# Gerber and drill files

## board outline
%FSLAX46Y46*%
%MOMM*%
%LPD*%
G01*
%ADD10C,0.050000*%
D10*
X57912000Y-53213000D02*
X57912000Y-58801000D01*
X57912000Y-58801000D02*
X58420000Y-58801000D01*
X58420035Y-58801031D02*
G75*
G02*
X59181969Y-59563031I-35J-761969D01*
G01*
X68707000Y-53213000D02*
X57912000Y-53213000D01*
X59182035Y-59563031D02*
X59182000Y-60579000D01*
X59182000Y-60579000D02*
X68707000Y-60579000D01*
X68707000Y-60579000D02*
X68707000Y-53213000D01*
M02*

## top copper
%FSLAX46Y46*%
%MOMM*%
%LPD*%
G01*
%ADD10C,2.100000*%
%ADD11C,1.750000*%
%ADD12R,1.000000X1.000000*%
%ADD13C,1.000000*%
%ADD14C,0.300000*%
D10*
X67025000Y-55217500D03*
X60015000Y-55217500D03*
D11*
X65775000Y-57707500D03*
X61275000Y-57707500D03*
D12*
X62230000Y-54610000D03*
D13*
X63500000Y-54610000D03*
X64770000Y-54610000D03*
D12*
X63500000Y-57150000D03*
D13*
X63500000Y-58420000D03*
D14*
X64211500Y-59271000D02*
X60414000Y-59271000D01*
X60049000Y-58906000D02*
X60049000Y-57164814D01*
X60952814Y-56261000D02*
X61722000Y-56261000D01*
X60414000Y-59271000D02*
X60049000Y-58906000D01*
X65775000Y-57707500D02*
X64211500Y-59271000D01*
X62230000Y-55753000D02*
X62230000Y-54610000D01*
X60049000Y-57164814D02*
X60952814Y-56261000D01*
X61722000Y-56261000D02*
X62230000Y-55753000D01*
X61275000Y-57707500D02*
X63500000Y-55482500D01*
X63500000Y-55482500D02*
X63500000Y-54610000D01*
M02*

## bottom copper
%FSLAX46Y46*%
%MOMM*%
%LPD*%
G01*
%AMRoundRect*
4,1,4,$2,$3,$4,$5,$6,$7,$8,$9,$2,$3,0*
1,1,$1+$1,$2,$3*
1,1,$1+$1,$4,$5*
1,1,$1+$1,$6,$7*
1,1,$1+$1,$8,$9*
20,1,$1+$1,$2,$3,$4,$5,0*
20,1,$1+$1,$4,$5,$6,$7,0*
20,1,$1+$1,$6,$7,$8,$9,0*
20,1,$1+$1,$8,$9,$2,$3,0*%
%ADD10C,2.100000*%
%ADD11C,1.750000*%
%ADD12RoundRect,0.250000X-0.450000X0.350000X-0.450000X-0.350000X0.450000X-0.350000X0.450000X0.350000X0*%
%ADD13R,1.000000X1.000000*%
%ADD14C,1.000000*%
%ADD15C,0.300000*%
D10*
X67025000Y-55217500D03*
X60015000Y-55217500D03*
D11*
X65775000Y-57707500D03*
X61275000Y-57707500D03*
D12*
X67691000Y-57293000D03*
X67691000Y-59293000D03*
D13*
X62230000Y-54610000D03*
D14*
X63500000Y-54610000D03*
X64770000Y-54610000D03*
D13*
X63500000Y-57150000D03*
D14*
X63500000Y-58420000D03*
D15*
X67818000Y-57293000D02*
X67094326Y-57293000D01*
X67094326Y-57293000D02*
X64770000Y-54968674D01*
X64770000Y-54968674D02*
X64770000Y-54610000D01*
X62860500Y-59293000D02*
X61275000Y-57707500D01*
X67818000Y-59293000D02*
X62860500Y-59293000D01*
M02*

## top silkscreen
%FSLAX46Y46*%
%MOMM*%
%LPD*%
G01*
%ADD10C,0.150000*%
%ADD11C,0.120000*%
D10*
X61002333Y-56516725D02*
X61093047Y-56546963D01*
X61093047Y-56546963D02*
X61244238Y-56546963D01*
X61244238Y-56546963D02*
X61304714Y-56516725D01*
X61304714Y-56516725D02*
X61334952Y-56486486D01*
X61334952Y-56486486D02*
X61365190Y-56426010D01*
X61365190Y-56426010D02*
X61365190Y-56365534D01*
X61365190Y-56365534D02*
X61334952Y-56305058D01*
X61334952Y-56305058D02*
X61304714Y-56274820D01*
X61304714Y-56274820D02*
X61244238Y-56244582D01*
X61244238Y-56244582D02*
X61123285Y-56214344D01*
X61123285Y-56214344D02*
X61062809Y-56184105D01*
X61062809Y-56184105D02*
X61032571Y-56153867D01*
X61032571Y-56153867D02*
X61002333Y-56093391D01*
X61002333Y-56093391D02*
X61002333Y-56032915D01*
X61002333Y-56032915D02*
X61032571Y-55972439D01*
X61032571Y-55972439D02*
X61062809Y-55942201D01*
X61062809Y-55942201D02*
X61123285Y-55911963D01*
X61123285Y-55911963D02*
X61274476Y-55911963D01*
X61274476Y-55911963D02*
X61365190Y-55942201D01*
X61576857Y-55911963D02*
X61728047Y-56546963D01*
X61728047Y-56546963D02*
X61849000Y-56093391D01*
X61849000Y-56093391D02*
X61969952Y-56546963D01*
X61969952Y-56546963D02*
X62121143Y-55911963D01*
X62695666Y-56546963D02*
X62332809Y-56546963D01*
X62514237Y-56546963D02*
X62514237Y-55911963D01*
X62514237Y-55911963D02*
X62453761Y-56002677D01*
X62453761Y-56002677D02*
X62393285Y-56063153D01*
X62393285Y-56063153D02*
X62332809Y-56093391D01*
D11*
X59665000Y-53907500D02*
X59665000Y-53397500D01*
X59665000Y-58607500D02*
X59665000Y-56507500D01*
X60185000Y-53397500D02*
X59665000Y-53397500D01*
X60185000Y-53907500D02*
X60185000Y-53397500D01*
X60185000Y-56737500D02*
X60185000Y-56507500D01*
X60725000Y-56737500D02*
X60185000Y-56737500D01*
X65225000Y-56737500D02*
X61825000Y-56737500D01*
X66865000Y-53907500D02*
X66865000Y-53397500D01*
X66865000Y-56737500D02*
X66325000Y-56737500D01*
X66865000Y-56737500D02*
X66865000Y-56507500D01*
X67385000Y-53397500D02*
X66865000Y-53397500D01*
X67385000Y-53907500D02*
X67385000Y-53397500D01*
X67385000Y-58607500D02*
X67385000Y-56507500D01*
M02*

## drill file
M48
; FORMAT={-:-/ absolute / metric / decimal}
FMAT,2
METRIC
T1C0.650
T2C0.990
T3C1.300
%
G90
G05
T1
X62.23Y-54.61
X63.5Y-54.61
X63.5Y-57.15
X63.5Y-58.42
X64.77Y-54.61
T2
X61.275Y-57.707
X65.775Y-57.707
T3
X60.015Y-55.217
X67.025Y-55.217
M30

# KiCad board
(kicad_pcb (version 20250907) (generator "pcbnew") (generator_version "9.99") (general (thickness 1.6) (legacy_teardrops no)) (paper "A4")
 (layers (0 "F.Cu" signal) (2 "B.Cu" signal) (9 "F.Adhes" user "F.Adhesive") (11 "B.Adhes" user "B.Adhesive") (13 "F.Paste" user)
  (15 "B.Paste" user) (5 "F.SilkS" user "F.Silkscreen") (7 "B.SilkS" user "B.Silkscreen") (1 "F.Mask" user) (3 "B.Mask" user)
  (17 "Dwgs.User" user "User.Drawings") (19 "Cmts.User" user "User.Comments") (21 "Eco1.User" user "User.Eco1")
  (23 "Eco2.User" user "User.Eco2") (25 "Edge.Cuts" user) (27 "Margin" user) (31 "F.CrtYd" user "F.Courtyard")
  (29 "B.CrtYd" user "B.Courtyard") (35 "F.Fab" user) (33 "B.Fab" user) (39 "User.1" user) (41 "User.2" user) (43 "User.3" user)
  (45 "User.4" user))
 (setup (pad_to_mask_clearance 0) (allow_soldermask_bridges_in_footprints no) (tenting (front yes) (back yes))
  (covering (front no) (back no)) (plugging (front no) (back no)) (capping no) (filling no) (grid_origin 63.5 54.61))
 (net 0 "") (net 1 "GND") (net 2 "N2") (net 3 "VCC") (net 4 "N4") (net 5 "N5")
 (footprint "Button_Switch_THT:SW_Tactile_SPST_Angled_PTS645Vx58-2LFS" (layer "F.Cu") (at 65.775 57.7075 180)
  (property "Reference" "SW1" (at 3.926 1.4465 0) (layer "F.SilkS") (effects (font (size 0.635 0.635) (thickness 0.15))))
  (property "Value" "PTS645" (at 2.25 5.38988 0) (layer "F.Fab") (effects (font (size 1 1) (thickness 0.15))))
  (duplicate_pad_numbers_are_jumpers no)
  (fp_line (start 6.11 3.8) (end 6.11 4.31) (stroke (width 0.12) (type solid)) (layer "F.SilkS"))
  (fp_line (start 6.11 -0.9) (end 6.11 1.2) (stroke (width 0.12) (type solid)) (layer "F.SilkS"))
  (fp_line (start 5.59 4.31) (end 6.11 4.31) (stroke (width 0.12) (type solid)) (layer "F.SilkS"))
  (fp_line (start 5.59 3.8) (end 5.59 4.31) (stroke (width 0.12) (type solid)) (layer "F.SilkS"))
  (fp_line (start 5.59 0.97) (end 5.59 1.2) (stroke (width 0.12) (type solid)) (layer "F.SilkS"))
  (fp_line (start 5.05 0.97) (end 5.59 0.97) (stroke (width 0.12) (type solid)) (layer "F.SilkS"))
  (fp_line (start 0.55 0.97) (end 3.95 0.97) (stroke (width 0.12) (type solid)) (layer "F.SilkS"))
  (fp_line (start -1.09 3.8) (end -1.09 4.31) (stroke (width 0.12) (type solid)) (layer "F.SilkS"))
  (fp_line (start -1.09 0.97) (end -0.55 0.97) (stroke (width 0.12) (type solid)) (layer "F.SilkS"))
  (fp_line (start -1.09 0.97) (end -1.09 1.2) (stroke (width 0.12) (type solid)) (layer "F.SilkS"))
  (fp_line (start -1.61 4.31) (end -1.09 4.31) (stroke (width 0.12) (type solid)) (layer "F.SilkS"))
  (fp_line (start -1.61 3.8) (end -1.61 4.31) (stroke (width 0.12) (type solid)) (layer "F.SilkS"))
  (fp_line (start -1.61 -0.9) (end -1.61 1.2) (stroke (width 0.12) (type solid)) (layer "F.SilkS"))
  (pad "" thru_hole circle (at -1.25 2.49 180) (size 2.1 2.1) (drill 1.3) (layers "*.Cu" "*.Mask") (remove_unused_layers no)
   (tenting (front none) (back none)))
  (pad "" thru_hole circle (at 5.76 2.49 180) (size 2.1 2.1) (drill 1.3) (layers "*.Cu" "*.Mask") (remove_unused_layers no)
   (tenting (front none) (back none)))
  (pad "1" thru_hole circle (at 0 0 180) (size 1.75 1.75) (drill 0.99) (layers "*.Cu" "*.Mask") (remove_unused_layers no) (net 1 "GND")
   (tenting (front none) (back none)))
  (pad "2" thru_hole circle (at 4.5 0 180) (size 1.75 1.75) (drill 0.99) (layers "*.Cu" "*.Mask") (remove_unused_layers no) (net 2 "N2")
   (tenting (front none) (back none))))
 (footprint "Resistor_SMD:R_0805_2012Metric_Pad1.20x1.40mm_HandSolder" (layer "B.Cu") (at 67.691 58.293 -90)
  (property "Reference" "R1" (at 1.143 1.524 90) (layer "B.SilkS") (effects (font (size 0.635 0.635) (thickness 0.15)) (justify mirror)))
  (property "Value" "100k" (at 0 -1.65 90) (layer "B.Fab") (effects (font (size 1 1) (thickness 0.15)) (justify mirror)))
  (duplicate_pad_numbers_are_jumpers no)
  (pad "1" smd roundrect (at -1 0 270) (size 1.2 1.4) (layers "B.Cu" "B.Mask" "B.Paste") (roundrect_rratio 0.208333) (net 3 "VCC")
   (tenting (front none) (back none)))
  (pad "2" smd roundrect (at 1 0 270) (size 1.2 1.4) (layers "B.Cu" "B.Mask" "B.Paste") (roundrect_rratio 0.208333) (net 2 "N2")
   (tenting (front none) (back none))))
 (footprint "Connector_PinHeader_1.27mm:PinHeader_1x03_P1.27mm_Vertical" (layer "B.Cu") (at 62.23 54.61 -90)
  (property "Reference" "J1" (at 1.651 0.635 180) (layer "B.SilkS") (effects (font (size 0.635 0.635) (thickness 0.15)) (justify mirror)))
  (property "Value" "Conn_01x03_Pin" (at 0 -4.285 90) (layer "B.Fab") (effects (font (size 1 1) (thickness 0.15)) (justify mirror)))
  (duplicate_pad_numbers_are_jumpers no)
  (pad "1" thru_hole rect (at 0 0 270) (size 1 1) (drill 0.65) (layers "*.Cu" "*.Mask") (remove_unused_layers no) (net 1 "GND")
   (tenting (front none) (back none)))
  (pad "2" thru_hole circle (at 0 -1.27 270) (size 1 1) (drill 0.65) (layers "*.Cu" "*.Mask") (remove_unused_layers no) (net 2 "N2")
   (tenting (front none) (back none)))
  (pad "3" thru_hole circle (at 0 -2.54 270) (size 1 1) (drill 0.65) (layers "*.Cu" "*.Mask") (remove_unused_layers no) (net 3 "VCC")
   (tenting (front none) (back none))))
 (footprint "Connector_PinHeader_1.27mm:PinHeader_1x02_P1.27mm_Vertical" (layer "B.Cu") (at 63.5 57.15 180)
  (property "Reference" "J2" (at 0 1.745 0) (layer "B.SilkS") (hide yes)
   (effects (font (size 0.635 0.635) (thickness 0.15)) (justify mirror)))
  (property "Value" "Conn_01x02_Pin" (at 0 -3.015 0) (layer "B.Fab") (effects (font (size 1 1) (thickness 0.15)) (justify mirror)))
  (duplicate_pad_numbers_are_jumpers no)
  (pad "1" thru_hole rect (at 0 0 180) (size 1 1) (drill 0.65) (layers "*.Cu" "*.Mask") (remove_unused_layers no) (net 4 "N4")
   (tenting (front none) (back none)))
  (pad "2" thru_hole circle (at 0 -1.27 180) (size 1 1) (drill 0.65) (layers "*.Cu" "*.Mask") (remove_unused_layers no) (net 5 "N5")
   (tenting (front none) (back none))))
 (gr_line (start 57.912 53.213) (end 57.912 58.801) (stroke (width 0.05) (type default)) (layer "Edge.Cuts"))
 (gr_line (start 57.912 58.801) (end 58.42 58.801) (stroke (width 0.05) (type default)) (layer "Edge.Cuts"))
 (gr_arc (start 58.420035 58.801031) (mid 58.95885 59.024216) (end 59.182035 59.563031) (stroke (width 0.05) (type default))
  (layer "Edge.Cuts"))
 (gr_line (start 68.707 53.213) (end 57.912 53.213) (stroke (width 0.05) (type default)) (layer "Edge.Cuts"))
 (gr_line (start 59.182035 59.563031) (end 59.182 60.579) (stroke (width 0.05) (type default)) (layer "Edge.Cuts"))
 (gr_line (start 59.182 60.579) (end 68.707 60.579) (stroke (width 0.05) (type default)) (layer "Edge.Cuts"))
 (gr_line (start 68.707 60.579) (end 68.707 53.213) (stroke (width 0.05) (type default)) (layer "Edge.Cuts"))
 (segment (start 67.818 57.293) (end 67.094326 57.293) (width 0.3) (layer "B.Cu") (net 3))
 (segment (start 67.094326 57.293) (end 64.77 54.968674) (width 0.3) (layer "B.Cu") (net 3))
 (segment (start 64.77 54.968674) (end 64.77 54.61) (width 0.3) (layer "B.Cu") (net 3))
 (segment (start 64.2115 59.271) (end 60.414 59.271) (width 0.3) (layer "F.Cu") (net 1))
 (segment (start 60.049 58.906) (end 60.049 57.164814) (width 0.3) (layer "F.Cu") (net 1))
 (segment (start 60.952814 56.261) (end 61.722 56.261) (width 0.3) (layer "F.Cu") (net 1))
 (segment (start 60.414 59.271) (end 60.049 58.906) (width 0.3) (layer "F.Cu") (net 1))
 (segment (start 65.775 57.7075) (end 64.2115 59.271) (width 0.3) (layer "F.Cu") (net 1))
 (segment (start 62.23 55.753) (end 62.23 54.61) (width 0.3) (layer "F.Cu") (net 1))
 (segment (start 60.049 57.164814) (end 60.952814 56.261) (width 0.3) (layer "F.Cu") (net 1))
 (segment (start 61.722 56.261) (end 62.23 55.753) (width 0.3) (layer "F.Cu") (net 1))
 (segment (start 61.275 57.7075) (end 63.5 55.4825) (width 0.3) (layer "F.Cu") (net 2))
 (segment (start 63.5 55.4825) (end 63.5 54.61) (width 0.3) (layer "F.Cu") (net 2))
 (segment (start 62.8605 59.293) (end 61.275 57.7075) (width 0.3) (layer "B.Cu") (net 2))
 (segment (start 67.818 59.293) (end 62.8605 59.293) (width 0.3) (layer "B.Cu") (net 2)))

